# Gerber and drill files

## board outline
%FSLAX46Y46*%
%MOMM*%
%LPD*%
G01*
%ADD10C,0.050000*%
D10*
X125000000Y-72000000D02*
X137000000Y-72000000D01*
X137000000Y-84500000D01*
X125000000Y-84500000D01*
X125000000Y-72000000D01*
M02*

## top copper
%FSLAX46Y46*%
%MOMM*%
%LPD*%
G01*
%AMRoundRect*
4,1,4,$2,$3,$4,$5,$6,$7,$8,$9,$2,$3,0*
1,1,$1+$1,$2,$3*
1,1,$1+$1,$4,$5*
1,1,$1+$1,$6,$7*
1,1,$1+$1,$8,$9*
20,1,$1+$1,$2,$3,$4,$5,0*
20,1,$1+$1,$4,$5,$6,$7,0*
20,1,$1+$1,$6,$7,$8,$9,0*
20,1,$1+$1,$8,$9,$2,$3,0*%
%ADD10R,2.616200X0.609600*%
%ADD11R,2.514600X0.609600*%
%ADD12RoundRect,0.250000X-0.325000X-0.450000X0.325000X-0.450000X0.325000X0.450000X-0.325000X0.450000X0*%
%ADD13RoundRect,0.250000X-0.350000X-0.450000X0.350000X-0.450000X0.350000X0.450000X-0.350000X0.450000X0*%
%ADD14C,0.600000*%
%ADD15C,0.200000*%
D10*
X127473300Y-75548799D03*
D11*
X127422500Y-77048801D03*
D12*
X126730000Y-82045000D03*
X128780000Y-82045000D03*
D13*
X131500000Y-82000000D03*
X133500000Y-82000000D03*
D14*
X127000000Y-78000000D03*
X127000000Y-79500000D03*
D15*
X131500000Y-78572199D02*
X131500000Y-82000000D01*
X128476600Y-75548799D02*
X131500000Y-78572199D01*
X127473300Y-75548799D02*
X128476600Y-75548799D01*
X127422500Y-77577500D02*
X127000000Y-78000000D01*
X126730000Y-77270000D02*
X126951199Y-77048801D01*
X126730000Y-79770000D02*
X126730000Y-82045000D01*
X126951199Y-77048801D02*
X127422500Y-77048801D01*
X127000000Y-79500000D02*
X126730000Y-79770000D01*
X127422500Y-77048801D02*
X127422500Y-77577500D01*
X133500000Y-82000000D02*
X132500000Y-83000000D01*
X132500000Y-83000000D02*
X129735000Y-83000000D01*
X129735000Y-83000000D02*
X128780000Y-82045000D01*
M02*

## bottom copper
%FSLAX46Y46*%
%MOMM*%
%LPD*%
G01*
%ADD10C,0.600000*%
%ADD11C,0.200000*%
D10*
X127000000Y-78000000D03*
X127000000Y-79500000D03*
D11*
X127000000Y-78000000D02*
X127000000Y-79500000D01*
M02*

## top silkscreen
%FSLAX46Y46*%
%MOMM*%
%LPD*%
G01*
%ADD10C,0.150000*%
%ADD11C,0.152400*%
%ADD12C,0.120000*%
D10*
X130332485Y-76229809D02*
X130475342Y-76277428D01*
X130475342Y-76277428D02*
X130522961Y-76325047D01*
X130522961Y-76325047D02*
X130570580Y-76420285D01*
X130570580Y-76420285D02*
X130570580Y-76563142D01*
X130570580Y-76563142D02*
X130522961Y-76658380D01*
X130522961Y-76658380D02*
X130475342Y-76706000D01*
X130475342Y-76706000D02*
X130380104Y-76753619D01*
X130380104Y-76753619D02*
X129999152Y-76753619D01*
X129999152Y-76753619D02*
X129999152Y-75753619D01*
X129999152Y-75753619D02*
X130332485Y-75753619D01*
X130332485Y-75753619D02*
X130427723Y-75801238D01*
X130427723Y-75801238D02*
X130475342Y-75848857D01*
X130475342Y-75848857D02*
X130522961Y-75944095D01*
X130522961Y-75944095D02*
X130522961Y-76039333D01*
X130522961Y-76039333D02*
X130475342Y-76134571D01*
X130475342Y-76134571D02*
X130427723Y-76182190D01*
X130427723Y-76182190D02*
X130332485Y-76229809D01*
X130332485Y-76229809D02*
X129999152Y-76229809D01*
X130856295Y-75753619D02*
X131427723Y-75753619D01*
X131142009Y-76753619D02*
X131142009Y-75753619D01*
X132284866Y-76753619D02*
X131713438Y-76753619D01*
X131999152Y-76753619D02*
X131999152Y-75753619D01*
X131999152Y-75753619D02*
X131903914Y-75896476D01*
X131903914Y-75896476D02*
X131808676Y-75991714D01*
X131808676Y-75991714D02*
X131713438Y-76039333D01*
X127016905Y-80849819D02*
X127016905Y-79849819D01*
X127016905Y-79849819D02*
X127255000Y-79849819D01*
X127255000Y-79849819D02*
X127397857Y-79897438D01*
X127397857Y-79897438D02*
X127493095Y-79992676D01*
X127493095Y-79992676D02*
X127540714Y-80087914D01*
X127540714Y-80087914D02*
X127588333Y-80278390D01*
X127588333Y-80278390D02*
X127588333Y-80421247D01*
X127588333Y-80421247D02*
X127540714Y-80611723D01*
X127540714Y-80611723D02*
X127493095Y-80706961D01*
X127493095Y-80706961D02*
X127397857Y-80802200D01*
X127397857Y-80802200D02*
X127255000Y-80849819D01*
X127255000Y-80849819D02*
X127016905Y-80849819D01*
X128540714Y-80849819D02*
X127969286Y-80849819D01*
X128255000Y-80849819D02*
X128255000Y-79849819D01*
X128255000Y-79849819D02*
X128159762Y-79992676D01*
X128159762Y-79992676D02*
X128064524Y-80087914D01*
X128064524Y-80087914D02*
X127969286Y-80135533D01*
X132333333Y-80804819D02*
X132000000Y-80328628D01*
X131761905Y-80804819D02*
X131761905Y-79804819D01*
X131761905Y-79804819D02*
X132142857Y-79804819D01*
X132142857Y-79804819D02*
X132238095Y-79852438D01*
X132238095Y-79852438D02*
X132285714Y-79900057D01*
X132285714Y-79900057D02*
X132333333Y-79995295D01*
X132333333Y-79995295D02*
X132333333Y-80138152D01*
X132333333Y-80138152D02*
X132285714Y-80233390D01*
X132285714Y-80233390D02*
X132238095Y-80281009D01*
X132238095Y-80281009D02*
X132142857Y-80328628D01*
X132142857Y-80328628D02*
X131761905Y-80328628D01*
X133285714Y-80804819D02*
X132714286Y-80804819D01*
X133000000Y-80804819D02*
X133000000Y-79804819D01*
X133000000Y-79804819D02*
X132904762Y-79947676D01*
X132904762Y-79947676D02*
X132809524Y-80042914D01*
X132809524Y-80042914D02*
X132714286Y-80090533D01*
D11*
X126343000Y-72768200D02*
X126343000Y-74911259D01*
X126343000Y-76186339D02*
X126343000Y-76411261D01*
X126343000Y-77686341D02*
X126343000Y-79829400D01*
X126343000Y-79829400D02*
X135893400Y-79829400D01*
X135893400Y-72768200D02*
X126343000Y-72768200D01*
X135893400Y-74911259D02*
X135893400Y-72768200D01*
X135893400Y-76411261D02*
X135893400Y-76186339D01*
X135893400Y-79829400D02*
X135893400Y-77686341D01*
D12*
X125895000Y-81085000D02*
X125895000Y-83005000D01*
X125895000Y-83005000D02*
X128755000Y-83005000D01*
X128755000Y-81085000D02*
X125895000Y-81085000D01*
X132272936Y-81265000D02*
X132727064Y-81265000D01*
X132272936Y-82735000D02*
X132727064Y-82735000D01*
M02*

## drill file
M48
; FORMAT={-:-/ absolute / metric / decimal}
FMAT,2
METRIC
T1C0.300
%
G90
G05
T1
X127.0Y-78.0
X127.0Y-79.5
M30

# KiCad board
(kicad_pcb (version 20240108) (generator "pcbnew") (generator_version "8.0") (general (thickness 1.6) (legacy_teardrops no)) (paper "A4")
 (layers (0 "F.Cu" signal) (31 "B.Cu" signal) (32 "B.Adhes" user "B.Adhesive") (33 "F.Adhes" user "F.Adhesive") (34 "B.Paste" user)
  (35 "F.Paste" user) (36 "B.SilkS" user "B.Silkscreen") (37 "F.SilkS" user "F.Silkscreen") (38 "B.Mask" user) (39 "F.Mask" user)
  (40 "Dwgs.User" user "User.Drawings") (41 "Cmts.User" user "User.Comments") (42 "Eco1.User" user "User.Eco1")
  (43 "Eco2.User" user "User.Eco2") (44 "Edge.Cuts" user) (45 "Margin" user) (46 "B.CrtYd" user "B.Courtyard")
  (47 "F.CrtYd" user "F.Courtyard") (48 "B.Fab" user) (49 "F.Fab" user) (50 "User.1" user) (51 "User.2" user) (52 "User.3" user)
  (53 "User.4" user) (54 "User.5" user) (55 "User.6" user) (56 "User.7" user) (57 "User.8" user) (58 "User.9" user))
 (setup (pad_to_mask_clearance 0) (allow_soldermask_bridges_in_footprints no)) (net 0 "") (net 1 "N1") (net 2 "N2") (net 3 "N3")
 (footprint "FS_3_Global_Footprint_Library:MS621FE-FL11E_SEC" (layer "F.Cu") (at 131.1182 76.2988)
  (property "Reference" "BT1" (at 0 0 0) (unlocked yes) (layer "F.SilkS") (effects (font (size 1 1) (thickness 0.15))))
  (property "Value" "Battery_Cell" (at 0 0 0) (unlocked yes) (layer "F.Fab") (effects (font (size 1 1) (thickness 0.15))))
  (fp_line (start -4.7752 -3.5306) (end -4.7752 -1.387541) (stroke (width 0.1524) (type solid)) (layer "F.SilkS"))
  (fp_line (start -4.7752 -0.112461) (end -4.7752 0.112461) (stroke (width 0.1524) (type solid)) (layer "F.SilkS"))
  (fp_line (start -4.7752 1.387541) (end -4.7752 3.5306) (stroke (width 0.1524) (type solid)) (layer "F.SilkS"))
  (fp_line (start -4.7752 3.5306) (end 4.7752 3.5306) (stroke (width 0.1524) (type solid)) (layer "F.SilkS"))
  (fp_line (start 4.7752 -3.5306) (end -4.7752 -3.5306) (stroke (width 0.1524) (type solid)) (layer "F.SilkS"))
  (fp_line (start 4.7752 -1.387541) (end 4.7752 -3.5306) (stroke (width 0.1524) (type solid)) (layer "F.SilkS"))
  (fp_line (start 4.7752 0.112461) (end 4.7752 -0.112461) (stroke (width 0.1524) (type solid)) (layer "F.SilkS"))
  (fp_line (start 4.7752 3.5306) (end 4.7752 1.387541) (stroke (width 0.1524) (type solid)) (layer "F.SilkS"))
  (pad "1" smd rect (at -3.6449 -0.750001) (size 2.6162 0.6096) (layers "F.Cu" "F.Paste" "F.Mask") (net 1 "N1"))
  (pad "2" smd rect (at -3.6957 0.750001) (size 2.5146 0.6096) (layers "F.Cu" "F.Paste" "F.Mask") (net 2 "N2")))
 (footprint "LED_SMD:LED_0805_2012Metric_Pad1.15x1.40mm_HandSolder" (layer "F.Cu") (at 127.755 82.045)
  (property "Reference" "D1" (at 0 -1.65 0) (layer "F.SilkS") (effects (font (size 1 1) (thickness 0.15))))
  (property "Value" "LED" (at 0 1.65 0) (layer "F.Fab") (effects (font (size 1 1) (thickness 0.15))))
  (fp_line (start -1.86 -0.96) (end -1.86 0.96) (stroke (width 0.12) (type solid)) (layer "F.SilkS"))
  (fp_line (start -1.86 0.96) (end 1 0.96) (stroke (width 0.12) (type solid)) (layer "F.SilkS"))
  (fp_line (start 1 -0.96) (end -1.86 -0.96) (stroke (width 0.12) (type solid)) (layer "F.SilkS"))
  (pad "1" smd roundrect (at -1.025 0) (size 1.15 1.4) (layers "F.Cu" "F.Paste" "F.Mask") (roundrect_rratio 0.217391) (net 2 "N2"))
  (pad "2" smd roundrect (at 1.025 0) (size 1.15 1.4) (layers "F.Cu" "F.Paste" "F.Mask") (roundrect_rratio 0.217391) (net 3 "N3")))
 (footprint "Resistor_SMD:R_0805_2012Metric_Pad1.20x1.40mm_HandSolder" (layer "F.Cu") (at 132.5 82)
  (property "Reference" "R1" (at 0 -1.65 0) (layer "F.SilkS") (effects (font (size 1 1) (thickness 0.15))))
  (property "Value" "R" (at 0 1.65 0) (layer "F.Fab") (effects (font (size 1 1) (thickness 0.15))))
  (fp_line (start -0.227064 -0.735) (end 0.227064 -0.735) (stroke (width 0.12) (type solid)) (layer "F.SilkS"))
  (fp_line (start -0.227064 0.735) (end 0.227064 0.735) (stroke (width 0.12) (type solid)) (layer "F.SilkS"))
  (pad "1" smd roundrect (at -1 0) (size 1.2 1.4) (layers "F.Cu" "F.Paste" "F.Mask") (roundrect_rratio 0.208333) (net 1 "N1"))
  (pad "2" smd roundrect (at 1 0) (size 1.2 1.4) (layers "F.Cu" "F.Paste" "F.Mask") (roundrect_rratio 0.208333) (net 3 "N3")))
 (gr_rect (start 125 72) (end 137 84.5) (stroke (width 0.05) (type default)) (fill none) (layer "Edge.Cuts"))
 (segment (start 131.5 78.572199) (end 131.5 82) (width 0.2) (layer "F.Cu") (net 1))
 (segment (start 128.4766 75.548799) (end 131.5 78.572199) (width 0.2) (layer "F.Cu") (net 1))
 (segment (start 127.4733 75.548799) (end 128.4766 75.548799) (width 0.2) (layer "F.Cu") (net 1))
 (segment (start 127.4225 77.5775) (end 127 78) (width 0.2) (layer "F.Cu") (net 2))
 (segment (start 126.73 77.27) (end 126.951199 77.048801) (width 0.2) (layer "F.Cu") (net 2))
 (segment (start 126.73 79.77) (end 126.73 82.045) (width 0.2) (layer "F.Cu") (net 2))
 (segment (start 126.951199 77.048801) (end 127.4225 77.048801) (width 0.2) (layer "F.Cu") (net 2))
 (segment (start 127 79.5) (end 126.73 79.77) (width 0.2) (layer "F.Cu") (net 2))
 (segment (start 127.4225 77.048801) (end 127.4225 77.5775) (width 0.2) (layer "F.Cu") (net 2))
 (via (at 127 78) (size 0.6) (drill 0.3) (layers "F.Cu" "B.Cu") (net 2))
 (via (at 127 79.5) (size 0.6) (drill 0.3) (layers "F.Cu" "B.Cu") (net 2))
 (segment (start 127 78) (end 127 79.5) (width 0.2) (layer "B.Cu") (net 2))
 (segment (start 133.5 82) (end 132.5 83) (width 0.2) (layer "F.Cu") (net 3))
 (segment (start 132.5 83) (end 129.735 83) (width 0.2) (layer "F.Cu") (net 3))
 (segment (start 129.735 83) (end 128.78 82.045) (width 0.2) (layer "F.Cu") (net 3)))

